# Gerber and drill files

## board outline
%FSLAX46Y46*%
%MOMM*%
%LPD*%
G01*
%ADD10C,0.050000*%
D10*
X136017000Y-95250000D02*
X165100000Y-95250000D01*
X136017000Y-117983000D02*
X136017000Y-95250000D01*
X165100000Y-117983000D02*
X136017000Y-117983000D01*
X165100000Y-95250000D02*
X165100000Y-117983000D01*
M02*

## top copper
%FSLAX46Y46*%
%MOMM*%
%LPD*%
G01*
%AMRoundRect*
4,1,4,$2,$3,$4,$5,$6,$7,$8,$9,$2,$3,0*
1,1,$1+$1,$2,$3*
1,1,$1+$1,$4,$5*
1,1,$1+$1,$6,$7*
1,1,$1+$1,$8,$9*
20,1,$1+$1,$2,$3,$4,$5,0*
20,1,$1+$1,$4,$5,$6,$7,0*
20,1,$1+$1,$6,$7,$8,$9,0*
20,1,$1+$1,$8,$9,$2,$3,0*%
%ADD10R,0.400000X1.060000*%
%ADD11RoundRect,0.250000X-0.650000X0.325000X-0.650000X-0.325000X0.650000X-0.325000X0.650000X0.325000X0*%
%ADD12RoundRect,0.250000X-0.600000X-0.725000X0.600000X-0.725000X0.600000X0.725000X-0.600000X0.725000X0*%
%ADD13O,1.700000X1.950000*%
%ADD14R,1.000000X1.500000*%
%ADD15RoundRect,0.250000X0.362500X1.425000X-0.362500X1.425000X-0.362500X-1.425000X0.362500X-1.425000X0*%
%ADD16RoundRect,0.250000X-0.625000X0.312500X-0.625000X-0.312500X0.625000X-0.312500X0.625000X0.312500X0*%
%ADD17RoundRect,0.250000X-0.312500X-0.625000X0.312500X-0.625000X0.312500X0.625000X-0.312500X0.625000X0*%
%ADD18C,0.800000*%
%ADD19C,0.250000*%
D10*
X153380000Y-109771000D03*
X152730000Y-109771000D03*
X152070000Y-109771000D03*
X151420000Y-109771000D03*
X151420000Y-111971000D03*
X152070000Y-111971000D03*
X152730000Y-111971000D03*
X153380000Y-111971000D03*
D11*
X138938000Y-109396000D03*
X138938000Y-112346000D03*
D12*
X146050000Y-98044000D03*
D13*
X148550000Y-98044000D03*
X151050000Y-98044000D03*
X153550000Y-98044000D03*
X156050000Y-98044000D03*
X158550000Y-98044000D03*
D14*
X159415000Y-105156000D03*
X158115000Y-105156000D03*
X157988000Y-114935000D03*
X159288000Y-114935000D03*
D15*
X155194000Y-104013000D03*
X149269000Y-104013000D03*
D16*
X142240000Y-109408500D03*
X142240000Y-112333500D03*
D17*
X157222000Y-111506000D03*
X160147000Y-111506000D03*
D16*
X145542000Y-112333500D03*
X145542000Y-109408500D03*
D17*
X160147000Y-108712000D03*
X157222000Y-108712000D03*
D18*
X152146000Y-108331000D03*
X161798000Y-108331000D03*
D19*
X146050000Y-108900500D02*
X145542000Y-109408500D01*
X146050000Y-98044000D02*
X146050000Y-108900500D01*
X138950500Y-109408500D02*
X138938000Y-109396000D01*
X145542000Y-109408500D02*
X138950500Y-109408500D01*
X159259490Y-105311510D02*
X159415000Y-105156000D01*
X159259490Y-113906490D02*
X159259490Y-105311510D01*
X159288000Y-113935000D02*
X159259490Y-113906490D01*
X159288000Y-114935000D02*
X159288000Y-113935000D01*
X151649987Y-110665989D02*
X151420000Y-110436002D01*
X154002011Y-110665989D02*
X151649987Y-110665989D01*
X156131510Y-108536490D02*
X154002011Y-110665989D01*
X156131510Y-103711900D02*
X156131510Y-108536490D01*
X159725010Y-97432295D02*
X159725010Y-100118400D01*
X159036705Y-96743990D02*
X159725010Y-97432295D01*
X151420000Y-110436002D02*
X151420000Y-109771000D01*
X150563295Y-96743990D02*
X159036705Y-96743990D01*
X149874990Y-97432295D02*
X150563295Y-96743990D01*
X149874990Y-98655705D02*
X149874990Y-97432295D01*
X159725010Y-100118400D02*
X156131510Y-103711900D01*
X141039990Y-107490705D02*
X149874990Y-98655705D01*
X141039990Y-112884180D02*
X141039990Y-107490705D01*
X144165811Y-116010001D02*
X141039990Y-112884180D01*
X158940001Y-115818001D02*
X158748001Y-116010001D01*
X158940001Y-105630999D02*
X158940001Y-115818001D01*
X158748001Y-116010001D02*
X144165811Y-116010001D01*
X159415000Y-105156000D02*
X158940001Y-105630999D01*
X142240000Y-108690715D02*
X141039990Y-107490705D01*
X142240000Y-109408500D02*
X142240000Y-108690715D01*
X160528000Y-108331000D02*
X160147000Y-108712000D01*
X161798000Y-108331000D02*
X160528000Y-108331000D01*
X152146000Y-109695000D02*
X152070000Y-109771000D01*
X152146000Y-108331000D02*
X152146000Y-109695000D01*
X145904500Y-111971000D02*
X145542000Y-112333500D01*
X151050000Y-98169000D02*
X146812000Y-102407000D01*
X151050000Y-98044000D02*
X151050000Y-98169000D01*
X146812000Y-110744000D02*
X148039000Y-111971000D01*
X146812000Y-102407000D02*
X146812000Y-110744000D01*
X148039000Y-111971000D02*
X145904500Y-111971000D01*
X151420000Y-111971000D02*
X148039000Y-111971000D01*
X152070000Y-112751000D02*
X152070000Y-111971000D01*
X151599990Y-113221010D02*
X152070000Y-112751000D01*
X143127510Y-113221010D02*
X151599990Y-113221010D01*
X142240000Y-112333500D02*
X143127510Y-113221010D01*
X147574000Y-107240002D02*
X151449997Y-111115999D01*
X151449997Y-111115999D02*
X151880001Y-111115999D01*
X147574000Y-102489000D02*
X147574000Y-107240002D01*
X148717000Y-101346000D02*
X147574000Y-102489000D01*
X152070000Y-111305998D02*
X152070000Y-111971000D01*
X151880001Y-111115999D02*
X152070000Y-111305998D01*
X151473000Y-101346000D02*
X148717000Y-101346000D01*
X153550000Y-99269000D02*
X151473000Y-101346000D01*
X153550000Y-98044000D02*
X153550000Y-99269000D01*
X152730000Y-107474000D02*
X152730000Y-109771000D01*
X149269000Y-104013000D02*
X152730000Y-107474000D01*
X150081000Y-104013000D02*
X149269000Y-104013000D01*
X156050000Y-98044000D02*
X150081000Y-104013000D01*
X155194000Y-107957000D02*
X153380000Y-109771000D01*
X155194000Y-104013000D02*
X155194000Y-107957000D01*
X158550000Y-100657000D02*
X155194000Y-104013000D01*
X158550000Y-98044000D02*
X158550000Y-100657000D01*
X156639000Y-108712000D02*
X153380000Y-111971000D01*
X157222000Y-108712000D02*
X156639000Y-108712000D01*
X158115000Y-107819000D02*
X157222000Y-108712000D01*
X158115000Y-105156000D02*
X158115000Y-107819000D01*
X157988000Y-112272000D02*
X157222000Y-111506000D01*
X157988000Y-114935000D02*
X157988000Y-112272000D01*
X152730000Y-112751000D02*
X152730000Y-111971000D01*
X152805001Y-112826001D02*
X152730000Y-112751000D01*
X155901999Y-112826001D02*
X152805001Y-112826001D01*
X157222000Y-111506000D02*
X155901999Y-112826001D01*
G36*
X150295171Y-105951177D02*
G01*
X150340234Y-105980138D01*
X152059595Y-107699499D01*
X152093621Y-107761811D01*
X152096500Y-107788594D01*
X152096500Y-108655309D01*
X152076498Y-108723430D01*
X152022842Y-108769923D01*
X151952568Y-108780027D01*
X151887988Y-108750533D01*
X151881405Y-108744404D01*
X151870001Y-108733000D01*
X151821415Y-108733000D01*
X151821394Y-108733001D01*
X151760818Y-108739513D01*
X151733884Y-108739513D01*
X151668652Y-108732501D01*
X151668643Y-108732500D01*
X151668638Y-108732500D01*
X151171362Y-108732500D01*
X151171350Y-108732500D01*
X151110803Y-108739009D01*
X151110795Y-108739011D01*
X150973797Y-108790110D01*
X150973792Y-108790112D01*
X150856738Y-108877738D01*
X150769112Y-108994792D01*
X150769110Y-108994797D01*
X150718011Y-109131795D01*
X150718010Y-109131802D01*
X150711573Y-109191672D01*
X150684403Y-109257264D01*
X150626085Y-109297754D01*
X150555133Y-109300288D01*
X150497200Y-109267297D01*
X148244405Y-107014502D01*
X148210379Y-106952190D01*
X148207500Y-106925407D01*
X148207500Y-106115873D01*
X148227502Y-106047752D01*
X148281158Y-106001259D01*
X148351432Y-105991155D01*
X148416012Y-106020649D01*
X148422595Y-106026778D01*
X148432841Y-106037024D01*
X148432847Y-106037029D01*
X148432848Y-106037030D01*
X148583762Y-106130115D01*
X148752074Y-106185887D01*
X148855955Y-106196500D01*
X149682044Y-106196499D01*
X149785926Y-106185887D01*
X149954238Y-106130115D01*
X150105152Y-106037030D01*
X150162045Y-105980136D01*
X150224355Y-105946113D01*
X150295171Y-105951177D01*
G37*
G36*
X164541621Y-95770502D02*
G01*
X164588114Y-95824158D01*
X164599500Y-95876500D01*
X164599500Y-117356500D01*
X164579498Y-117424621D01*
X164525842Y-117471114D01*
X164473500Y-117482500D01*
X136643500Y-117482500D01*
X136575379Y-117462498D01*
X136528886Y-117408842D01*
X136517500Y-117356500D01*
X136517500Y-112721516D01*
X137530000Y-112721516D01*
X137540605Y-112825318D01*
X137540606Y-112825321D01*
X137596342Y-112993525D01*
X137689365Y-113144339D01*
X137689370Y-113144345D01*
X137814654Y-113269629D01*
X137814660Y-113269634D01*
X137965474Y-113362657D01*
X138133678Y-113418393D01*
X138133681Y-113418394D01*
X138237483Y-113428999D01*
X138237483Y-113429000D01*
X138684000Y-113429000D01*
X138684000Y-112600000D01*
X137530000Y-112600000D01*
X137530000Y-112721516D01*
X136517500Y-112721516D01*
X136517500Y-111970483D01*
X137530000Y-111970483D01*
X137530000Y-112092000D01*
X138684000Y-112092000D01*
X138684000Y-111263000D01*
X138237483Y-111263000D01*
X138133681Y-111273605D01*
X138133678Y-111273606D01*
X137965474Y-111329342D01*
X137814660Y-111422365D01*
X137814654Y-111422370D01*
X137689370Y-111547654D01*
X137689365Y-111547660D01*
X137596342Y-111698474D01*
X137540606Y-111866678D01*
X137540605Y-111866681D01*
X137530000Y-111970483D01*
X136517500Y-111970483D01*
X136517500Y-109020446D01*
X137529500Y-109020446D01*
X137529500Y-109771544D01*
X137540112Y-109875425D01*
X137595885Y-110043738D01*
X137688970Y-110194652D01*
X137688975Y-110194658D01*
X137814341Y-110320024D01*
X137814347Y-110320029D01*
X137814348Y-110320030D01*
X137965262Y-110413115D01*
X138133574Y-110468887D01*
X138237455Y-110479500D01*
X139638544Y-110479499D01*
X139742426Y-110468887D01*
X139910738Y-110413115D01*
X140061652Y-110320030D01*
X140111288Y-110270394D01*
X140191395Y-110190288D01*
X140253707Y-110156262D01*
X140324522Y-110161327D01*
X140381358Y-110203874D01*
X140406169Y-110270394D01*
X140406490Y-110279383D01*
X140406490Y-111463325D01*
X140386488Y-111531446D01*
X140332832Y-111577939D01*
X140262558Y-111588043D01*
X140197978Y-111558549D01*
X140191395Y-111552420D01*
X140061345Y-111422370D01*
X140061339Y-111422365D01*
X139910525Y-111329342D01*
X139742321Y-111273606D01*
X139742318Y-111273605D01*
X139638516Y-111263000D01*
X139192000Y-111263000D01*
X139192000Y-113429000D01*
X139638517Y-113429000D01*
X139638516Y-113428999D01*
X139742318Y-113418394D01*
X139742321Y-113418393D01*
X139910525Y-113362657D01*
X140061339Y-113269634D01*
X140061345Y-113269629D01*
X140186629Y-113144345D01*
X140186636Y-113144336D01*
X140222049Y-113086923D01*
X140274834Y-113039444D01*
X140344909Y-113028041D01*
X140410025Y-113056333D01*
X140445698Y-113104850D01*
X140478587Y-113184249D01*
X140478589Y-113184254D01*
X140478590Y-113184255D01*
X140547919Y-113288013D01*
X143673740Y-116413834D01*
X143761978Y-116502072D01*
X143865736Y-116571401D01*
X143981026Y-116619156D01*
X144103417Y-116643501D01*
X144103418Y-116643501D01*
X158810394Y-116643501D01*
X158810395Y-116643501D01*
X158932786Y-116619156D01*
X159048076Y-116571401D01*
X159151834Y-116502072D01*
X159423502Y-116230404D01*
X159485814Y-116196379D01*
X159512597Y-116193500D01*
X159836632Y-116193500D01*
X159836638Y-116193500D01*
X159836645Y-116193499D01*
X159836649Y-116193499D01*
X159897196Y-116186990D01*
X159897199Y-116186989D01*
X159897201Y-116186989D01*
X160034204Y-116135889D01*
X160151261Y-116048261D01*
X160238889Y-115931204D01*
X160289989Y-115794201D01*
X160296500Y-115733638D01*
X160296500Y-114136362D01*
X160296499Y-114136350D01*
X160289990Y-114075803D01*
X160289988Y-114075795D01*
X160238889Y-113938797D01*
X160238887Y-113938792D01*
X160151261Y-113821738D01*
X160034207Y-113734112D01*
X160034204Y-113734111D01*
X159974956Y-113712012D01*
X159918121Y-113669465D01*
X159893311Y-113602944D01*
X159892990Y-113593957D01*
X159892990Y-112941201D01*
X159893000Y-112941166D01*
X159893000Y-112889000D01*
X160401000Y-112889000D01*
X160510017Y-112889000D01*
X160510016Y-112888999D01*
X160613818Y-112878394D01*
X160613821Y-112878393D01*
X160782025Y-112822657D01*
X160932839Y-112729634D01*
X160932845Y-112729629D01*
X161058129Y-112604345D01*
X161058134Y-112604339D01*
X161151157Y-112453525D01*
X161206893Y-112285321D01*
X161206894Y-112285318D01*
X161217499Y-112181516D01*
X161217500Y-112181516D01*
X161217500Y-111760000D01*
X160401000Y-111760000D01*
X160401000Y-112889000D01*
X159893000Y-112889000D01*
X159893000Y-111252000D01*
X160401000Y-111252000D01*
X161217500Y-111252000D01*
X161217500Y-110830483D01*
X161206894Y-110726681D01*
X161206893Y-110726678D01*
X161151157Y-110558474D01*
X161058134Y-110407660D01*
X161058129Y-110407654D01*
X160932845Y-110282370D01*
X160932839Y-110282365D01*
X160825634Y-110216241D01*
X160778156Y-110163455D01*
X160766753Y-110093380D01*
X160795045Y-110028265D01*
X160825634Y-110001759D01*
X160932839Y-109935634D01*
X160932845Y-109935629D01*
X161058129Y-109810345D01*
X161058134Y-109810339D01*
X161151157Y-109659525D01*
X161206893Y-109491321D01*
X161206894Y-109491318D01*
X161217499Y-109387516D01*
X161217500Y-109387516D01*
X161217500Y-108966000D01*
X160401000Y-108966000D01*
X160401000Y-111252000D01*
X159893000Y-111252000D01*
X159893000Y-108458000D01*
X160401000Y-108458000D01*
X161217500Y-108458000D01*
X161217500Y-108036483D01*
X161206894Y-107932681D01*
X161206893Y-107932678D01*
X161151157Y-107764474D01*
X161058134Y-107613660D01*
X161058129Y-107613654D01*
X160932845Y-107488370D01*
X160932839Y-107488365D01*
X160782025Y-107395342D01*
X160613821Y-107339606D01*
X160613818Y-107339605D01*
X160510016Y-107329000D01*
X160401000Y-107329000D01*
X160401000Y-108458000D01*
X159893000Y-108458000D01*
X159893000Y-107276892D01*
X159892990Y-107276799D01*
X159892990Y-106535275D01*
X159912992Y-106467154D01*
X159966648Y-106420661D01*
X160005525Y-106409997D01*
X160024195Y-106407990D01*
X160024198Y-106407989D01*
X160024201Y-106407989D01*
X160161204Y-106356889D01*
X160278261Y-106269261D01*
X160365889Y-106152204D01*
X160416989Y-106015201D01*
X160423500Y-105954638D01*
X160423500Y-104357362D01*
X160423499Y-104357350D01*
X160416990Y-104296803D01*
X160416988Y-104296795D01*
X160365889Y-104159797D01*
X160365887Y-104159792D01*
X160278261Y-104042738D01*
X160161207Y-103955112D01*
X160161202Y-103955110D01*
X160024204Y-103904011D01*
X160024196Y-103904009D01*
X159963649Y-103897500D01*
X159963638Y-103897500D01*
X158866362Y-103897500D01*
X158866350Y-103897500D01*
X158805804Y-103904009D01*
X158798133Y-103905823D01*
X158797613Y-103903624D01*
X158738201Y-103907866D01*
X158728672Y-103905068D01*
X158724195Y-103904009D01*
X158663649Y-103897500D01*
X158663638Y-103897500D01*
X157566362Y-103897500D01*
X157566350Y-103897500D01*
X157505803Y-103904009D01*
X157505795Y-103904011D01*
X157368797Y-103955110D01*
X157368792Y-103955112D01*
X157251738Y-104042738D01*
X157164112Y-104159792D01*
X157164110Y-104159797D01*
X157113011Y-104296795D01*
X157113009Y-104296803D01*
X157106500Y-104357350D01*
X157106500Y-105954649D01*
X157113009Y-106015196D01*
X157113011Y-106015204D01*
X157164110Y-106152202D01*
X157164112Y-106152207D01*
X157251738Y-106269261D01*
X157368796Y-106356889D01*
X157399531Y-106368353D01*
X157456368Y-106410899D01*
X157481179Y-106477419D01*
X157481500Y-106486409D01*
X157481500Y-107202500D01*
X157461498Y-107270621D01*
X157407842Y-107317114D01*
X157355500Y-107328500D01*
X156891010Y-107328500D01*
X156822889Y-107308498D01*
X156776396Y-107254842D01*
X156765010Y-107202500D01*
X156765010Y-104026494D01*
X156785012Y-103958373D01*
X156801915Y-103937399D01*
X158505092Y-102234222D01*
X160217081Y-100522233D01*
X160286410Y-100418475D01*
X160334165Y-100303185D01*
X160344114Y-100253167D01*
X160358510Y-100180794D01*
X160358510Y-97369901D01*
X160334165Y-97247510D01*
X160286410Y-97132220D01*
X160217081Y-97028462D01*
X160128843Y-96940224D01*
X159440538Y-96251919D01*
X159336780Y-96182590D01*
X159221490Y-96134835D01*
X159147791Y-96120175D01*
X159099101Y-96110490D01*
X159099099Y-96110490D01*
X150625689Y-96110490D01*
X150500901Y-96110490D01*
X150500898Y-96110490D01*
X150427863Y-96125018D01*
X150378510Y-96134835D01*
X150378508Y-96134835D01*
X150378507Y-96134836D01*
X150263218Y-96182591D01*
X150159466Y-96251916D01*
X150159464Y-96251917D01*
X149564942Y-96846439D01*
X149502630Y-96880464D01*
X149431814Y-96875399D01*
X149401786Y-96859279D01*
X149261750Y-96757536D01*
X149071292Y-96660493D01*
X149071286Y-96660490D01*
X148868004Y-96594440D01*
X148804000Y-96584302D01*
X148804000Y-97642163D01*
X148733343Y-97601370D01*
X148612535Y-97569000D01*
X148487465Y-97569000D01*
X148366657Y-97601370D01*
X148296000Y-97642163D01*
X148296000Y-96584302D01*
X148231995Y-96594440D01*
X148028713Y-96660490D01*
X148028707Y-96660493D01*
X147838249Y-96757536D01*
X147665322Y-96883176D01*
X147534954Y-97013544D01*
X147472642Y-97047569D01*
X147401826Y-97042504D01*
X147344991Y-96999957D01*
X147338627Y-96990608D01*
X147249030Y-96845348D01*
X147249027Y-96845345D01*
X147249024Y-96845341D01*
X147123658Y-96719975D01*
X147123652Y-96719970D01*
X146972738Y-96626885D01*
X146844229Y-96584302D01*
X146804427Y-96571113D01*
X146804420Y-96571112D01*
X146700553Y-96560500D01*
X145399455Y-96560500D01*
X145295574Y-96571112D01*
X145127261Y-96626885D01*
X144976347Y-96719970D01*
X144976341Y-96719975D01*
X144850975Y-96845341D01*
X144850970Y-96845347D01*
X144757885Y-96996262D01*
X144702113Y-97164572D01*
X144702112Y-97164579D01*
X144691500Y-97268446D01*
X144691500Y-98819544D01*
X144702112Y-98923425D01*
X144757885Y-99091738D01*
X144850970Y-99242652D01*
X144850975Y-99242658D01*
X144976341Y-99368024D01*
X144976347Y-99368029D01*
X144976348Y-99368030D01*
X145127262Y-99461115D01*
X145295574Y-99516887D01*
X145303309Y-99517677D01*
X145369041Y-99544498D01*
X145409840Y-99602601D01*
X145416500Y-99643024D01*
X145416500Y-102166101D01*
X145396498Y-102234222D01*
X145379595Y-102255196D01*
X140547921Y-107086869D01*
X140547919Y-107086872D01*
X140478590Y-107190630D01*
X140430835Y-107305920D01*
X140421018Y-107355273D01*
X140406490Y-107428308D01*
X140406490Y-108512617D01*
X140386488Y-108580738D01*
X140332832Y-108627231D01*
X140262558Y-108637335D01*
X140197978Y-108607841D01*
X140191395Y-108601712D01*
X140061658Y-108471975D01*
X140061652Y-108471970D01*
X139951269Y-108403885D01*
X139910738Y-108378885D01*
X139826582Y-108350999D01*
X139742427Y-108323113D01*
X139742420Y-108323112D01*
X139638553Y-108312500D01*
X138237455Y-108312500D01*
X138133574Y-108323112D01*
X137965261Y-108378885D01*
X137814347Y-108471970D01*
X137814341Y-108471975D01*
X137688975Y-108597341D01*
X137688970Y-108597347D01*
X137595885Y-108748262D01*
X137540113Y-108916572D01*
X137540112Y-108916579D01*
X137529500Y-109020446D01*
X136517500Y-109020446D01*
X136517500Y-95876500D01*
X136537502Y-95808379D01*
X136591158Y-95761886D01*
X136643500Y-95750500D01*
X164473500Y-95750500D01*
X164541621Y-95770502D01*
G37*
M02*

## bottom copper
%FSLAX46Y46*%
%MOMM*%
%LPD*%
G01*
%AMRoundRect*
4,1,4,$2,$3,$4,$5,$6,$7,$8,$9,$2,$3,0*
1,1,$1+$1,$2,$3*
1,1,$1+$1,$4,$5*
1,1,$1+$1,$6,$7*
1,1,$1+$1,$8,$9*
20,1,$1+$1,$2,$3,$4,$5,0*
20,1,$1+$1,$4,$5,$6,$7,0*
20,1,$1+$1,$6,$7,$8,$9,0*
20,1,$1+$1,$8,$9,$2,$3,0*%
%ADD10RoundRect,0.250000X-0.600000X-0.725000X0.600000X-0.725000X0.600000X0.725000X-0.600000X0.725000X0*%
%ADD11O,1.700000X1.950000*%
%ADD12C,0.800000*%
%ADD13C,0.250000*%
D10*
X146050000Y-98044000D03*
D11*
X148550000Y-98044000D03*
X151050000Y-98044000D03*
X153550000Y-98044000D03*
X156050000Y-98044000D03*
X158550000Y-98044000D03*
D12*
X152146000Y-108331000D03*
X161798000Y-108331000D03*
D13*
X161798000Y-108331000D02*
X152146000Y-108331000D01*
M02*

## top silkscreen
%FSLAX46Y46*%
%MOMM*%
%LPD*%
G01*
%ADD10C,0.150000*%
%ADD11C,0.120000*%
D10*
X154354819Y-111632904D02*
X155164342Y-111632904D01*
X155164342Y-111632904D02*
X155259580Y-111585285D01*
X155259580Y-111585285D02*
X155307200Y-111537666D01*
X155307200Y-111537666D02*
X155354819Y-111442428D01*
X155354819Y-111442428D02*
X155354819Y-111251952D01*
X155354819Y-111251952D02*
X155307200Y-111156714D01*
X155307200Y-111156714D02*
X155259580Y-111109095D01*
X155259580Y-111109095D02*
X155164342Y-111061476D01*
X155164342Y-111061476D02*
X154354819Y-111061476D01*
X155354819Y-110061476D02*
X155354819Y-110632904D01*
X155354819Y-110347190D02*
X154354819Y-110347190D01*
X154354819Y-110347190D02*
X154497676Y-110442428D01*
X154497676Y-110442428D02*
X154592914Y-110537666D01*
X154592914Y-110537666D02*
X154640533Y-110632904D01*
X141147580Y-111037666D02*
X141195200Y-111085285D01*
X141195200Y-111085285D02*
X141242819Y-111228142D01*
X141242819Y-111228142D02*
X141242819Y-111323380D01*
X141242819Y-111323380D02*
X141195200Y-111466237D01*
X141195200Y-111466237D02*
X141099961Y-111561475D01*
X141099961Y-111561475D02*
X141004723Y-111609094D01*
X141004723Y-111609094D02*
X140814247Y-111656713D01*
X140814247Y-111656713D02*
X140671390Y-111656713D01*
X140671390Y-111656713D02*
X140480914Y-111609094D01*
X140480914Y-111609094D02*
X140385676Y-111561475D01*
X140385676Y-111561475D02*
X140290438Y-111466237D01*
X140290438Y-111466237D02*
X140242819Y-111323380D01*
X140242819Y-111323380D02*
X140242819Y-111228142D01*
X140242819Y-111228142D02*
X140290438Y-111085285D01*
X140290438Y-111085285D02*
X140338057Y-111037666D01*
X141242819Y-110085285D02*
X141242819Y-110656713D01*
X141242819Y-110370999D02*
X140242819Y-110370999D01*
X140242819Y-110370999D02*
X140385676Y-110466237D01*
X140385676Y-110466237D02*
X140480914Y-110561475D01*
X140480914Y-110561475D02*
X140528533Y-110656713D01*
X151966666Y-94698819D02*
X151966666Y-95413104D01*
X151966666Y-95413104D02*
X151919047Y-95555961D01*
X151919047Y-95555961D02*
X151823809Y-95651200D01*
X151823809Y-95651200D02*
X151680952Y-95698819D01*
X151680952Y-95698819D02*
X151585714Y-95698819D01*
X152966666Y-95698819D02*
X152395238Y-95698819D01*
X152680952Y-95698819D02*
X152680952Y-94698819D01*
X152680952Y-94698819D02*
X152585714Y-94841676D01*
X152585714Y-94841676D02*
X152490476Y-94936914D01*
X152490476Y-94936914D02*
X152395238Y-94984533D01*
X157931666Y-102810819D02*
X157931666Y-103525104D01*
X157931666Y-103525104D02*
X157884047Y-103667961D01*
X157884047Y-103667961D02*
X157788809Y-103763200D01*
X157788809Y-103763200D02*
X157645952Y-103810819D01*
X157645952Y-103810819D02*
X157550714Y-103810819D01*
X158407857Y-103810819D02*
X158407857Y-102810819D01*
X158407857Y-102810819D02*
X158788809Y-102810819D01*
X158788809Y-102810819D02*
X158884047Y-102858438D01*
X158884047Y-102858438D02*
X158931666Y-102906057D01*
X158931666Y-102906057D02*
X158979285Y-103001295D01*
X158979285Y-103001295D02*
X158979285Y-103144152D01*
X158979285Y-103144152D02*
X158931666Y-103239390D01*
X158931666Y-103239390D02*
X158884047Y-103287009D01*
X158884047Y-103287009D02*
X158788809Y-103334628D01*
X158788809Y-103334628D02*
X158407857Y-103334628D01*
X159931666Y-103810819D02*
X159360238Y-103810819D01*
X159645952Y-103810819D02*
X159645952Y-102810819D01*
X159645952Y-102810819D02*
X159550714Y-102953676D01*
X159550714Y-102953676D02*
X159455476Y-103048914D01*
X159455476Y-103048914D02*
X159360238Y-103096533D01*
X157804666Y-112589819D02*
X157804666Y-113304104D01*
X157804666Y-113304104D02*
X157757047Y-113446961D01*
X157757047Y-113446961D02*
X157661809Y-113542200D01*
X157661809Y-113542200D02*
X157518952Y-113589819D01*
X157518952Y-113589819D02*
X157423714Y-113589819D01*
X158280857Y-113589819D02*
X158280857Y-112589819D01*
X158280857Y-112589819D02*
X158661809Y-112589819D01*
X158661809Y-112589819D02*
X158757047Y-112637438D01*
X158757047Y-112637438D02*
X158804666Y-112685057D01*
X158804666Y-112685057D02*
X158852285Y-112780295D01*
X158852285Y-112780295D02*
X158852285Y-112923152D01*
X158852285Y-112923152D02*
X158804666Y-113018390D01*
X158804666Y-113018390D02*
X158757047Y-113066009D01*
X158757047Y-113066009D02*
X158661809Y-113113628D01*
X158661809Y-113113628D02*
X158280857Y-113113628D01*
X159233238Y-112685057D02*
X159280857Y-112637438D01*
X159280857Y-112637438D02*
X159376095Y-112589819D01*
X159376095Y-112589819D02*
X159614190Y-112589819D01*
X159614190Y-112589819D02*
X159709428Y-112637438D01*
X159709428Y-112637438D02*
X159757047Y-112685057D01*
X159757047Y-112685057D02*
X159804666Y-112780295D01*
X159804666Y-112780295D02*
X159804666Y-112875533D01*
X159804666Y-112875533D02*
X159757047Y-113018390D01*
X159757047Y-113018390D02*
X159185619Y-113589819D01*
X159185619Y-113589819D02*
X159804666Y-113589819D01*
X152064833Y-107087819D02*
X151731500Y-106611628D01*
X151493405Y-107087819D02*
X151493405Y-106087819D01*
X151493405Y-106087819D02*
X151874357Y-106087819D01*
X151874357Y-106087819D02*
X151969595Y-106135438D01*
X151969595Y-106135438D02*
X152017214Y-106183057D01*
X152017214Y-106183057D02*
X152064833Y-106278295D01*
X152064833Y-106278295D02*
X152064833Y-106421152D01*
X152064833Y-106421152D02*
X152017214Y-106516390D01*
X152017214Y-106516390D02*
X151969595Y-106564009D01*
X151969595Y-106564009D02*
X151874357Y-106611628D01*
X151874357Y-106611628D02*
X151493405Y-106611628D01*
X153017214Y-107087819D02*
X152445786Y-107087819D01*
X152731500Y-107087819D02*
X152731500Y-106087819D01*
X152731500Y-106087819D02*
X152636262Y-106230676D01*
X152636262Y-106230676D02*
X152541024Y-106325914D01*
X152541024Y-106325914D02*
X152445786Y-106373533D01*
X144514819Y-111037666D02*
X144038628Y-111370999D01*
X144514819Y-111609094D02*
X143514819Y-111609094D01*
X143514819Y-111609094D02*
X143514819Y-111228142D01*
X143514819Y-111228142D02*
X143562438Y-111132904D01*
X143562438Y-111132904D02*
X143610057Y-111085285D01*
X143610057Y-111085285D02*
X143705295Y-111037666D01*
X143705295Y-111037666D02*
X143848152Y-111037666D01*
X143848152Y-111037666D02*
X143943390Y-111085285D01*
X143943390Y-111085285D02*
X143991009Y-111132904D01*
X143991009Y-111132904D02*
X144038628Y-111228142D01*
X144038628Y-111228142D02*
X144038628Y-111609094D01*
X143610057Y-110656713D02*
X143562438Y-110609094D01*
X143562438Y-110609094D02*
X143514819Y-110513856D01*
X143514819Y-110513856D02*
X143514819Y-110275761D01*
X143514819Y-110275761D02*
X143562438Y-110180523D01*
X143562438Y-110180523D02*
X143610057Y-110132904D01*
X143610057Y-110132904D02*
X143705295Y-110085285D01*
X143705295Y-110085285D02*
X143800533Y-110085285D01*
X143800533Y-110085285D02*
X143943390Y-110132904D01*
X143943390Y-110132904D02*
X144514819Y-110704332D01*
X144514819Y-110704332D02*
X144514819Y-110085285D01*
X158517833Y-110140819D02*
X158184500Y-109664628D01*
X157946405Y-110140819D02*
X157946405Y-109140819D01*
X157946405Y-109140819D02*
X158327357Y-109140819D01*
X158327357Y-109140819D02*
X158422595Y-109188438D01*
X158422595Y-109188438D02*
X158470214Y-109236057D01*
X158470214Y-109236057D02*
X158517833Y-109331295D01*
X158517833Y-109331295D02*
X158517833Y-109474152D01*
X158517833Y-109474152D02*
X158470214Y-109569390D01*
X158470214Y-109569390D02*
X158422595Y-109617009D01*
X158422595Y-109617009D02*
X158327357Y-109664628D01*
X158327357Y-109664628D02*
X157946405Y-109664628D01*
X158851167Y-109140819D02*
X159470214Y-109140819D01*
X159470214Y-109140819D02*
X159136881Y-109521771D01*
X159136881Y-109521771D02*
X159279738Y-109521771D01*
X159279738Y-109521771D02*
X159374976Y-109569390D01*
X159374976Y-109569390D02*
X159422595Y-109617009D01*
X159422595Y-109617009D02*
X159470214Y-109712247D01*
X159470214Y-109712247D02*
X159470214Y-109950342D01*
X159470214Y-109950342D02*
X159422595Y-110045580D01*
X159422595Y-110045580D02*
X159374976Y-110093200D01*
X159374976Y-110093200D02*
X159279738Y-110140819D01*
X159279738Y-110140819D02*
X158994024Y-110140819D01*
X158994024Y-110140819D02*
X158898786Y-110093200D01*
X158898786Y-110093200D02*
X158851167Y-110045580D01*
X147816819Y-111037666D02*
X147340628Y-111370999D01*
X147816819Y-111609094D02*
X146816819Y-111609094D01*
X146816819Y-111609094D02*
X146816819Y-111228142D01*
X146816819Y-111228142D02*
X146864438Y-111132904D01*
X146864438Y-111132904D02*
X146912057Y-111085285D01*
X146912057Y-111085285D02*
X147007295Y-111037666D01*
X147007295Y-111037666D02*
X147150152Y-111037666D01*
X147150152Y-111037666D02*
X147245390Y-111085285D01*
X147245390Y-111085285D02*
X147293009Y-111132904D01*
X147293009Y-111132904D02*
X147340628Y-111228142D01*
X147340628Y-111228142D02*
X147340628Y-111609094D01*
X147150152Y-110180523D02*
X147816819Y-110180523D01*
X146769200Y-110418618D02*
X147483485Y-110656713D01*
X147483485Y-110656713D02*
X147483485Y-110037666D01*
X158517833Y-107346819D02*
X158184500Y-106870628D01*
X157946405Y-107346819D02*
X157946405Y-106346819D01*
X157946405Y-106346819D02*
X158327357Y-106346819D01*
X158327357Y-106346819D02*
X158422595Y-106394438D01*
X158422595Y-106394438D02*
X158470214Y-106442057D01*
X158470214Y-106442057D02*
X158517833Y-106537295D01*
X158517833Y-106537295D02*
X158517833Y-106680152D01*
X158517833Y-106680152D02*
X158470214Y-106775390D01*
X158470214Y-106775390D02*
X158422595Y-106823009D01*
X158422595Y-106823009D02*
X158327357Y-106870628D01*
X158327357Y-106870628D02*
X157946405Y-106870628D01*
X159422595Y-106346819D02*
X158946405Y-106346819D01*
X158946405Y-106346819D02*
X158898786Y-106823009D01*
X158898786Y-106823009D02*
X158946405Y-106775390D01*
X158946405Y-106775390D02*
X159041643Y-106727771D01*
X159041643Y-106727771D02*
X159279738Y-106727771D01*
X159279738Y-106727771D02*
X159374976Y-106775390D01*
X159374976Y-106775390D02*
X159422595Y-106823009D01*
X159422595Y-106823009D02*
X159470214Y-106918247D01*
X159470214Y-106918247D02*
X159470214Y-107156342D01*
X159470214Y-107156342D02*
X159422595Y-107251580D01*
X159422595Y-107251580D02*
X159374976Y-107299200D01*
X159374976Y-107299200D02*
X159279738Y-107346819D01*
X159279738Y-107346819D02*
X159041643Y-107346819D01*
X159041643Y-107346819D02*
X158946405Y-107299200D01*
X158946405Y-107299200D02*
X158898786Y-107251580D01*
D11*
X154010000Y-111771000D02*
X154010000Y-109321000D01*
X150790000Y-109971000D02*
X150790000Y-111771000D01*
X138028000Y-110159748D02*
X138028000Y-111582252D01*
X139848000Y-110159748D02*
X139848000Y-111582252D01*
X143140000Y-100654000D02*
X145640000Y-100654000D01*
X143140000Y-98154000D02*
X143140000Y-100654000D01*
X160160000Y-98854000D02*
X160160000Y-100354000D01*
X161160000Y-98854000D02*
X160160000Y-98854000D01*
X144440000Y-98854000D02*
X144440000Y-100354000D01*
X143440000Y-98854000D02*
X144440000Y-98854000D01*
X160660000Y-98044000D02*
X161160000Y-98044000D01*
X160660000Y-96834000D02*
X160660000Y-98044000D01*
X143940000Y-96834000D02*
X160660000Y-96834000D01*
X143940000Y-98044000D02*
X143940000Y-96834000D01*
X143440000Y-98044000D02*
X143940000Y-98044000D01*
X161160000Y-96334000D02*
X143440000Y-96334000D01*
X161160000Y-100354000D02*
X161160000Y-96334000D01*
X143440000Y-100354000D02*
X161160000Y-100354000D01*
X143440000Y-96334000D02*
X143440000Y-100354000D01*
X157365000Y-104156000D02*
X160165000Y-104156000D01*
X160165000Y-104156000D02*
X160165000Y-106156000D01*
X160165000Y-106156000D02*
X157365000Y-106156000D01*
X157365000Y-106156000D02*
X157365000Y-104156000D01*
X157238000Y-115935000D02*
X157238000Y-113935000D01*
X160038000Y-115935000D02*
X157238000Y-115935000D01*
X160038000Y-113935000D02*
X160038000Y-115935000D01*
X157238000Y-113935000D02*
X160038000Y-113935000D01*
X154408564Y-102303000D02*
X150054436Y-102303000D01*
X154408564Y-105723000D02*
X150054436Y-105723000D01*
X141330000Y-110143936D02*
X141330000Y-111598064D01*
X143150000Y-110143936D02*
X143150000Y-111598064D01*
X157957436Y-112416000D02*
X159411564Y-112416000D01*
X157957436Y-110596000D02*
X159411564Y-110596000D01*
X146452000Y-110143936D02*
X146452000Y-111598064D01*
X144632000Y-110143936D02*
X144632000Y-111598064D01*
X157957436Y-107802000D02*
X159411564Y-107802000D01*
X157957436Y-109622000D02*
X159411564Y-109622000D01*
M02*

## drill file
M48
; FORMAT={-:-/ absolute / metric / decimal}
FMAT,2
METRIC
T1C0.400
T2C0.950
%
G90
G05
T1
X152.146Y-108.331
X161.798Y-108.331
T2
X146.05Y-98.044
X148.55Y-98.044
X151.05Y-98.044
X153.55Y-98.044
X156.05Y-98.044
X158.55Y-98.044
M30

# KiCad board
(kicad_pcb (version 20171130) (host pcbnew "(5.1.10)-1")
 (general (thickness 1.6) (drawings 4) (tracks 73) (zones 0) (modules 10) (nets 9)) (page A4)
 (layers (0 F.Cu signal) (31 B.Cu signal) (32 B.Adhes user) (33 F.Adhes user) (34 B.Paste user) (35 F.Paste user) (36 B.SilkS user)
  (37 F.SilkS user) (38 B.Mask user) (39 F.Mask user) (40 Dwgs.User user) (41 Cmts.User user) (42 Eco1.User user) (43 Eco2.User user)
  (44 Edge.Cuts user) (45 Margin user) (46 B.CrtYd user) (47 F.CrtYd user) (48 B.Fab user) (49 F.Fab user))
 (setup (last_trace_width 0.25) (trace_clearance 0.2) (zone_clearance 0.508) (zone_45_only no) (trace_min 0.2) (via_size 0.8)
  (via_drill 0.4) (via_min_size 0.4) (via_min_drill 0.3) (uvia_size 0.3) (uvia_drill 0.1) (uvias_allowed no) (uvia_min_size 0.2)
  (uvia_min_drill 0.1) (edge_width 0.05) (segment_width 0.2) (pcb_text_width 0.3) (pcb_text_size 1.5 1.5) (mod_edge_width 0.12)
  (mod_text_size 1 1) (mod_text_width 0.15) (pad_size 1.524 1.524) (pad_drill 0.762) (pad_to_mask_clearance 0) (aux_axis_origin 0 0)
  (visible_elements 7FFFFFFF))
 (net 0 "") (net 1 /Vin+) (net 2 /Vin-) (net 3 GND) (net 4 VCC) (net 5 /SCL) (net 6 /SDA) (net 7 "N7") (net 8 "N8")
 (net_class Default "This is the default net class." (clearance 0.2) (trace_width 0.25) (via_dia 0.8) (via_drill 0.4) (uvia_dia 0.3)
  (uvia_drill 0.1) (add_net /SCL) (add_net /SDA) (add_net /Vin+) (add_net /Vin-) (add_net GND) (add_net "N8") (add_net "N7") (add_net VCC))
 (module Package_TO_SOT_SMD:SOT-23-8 (layer F.Cu) (at 152.4 110.871 270)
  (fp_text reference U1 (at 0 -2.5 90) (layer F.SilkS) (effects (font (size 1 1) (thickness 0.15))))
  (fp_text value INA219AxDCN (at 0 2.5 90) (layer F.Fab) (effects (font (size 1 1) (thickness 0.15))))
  (fp_line (start 0.9 -1.61) (end -1.55 -1.61) (layer F.SilkS) (width 0.12))
  (fp_line (start -0.9 1.61) (end 0.9 1.61) (layer F.SilkS) (width 0.12))
  (pad 1 smd rect (at -1.1 -0.98 270) (size 1.06 0.4) (layers F.Cu F.Paste F.Mask) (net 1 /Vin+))
  (pad 2 smd rect (at -1.1 -0.33 270) (size 1.06 0.4) (layers F.Cu F.Paste F.Mask) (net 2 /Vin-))
  (pad 3 smd rect (at -1.1 0.33 270) (size 1.06 0.4) (layers F.Cu F.Paste F.Mask) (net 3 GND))
  (pad 4 smd rect (at -1.1 0.98 270) (size 1.06 0.4) (layers F.Cu F.Paste F.Mask) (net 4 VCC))
  (pad 5 smd rect (at 1.1 0.98 270) (size 1.06 0.4) (layers F.Cu F.Paste F.Mask) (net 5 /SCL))
  (pad 6 smd rect (at 1.1 0.33 270) (size 1.06 0.4) (layers F.Cu F.Paste F.Mask) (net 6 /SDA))
  (pad 7 smd rect (at 1.1 -0.33 270) (size 1.06 0.4) (layers F.Cu F.Paste F.Mask) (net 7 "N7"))
  (pad 8 smd rect (at 1.1 -0.98 270) (size 1.06 0.4) (layers F.Cu F.Paste F.Mask) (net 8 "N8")))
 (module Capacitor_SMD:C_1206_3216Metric (layer F.Cu) (at 138.938 110.871 270)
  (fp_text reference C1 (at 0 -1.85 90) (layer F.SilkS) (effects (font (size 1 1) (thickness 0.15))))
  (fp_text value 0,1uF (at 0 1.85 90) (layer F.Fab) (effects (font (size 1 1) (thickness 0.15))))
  (fp_line (start -0.711252 0.91) (end 0.711252 0.91) (layer F.SilkS) (width 0.12))
  (fp_line (start -0.711252 -0.91) (end 0.711252 -0.91) (layer F.SilkS) (width 0.12))
  (pad 1 smd roundrect (at -1.475 0 270) (size 1.15 1.8) (layers F.Cu F.Paste F.Mask) (roundrect_rratio 0.217391) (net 4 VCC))
  (pad 2 smd roundrect (at 1.475 0 270) (size 1.15 1.8) (layers F.Cu F.Paste F.Mask) (roundrect_rratio 0.217391) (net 3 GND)))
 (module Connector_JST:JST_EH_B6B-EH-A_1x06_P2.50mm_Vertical (layer F.Cu) (at 146.05 98.044)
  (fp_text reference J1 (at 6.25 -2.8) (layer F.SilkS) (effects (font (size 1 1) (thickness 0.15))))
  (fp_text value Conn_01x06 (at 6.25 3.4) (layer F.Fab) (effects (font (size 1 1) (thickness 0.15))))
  (fp_line (start -2.91 2.61) (end -0.41 2.61) (layer F.SilkS) (width 0.12))
  (fp_line (start -2.91 0.11) (end -2.91 2.61) (layer F.SilkS) (width 0.12))
  (fp_line (start 14.11 0.81) (end 14.11 2.31) (layer F.SilkS) (width 0.12))
  (fp_line (start 15.11 0.81) (end 14.11 0.81) (layer F.SilkS) (width 0.12))
  (fp_line (start -1.61 0.81) (end -1.61 2.31) (layer F.SilkS) (width 0.12))
  (fp_line (start -2.61 0.81) (end -1.61 0.81) (layer F.SilkS) (width 0.12))
  (fp_line (start 14.61 0) (end 15.11 0) (layer F.SilkS) (width 0.12))
  (fp_line (start 14.61 -1.21) (end 14.61 0) (layer F.SilkS) (width 0.12))
  (fp_line (start -2.11 -1.21) (end 14.61 -1.21) (layer F.SilkS) (width 0.12))
  (fp_line (start -2.11 0) (end -2.11 -1.21) (layer F.SilkS) (width 0.12))
  (fp_line (start -2.61 0) (end -2.11 0) (layer F.SilkS) (width 0.12))
  (fp_line (start 15.11 -1.71) (end -2.61 -1.71) (layer F.SilkS) (width 0.12))
  (fp_line (start 15.11 2.31) (end 15.11 -1.71) (layer F.SilkS) (width 0.12))
  (fp_line (start -2.61 2.31) (end 15.11 2.31) (layer F.SilkS) (width 0.12))
  (fp_line (start -2.61 -1.71) (end -2.61 2.31) (layer F.SilkS) (width 0.12))
  (pad 1 thru_hole roundrect (at 0 0) (size 1.7 1.95) (drill 0.95) (layers *.Cu *.Mask) (roundrect_rratio 0.147059) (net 4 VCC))
  (pad 2 thru_hole oval (at 2.5 0) (size 1.7 1.95) (drill 0.95) (layers *.Cu *.Mask) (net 3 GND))
  (pad 3 thru_hole oval (at 5 0) (size 1.7 1.95) (drill 0.95) (layers *.Cu *.Mask) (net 5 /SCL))
  (pad 4 thru_hole oval (at 7.5 0) (size 1.7 1.95) (drill 0.95) (layers *.Cu *.Mask) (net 6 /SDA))
  (pad 5 thru_hole oval (at 10 0) (size 1.7 1.95) (drill 0.95) (layers *.Cu *.Mask) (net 2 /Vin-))
  (pad 6 thru_hole oval (at 12.5 0) (size 1.7 1.95) (drill 0.95) (layers *.Cu *.Mask) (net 1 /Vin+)))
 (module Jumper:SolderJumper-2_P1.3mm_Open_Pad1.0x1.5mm (layer F.Cu) (at 158.765 105.156)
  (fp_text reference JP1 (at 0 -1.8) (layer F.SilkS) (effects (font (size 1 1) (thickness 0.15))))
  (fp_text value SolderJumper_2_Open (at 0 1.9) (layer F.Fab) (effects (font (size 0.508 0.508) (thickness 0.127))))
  (fp_line (start -1.4 -1) (end 1.4 -1) (layer F.SilkS) (width 0.12))
  (fp_line (start 1.4 -1) (end 1.4 1) (layer F.SilkS) (width 0.12))
  (fp_line (start 1.4 1) (end -1.4 1) (layer F.SilkS) (width 0.12))
  (fp_line (start -1.4 1) (end -1.4 -1) (layer F.SilkS) (width 0.12))
  (pad 2 smd rect (at 0.65 0) (size 1 1.5) (layers F.Cu F.Mask) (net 4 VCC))
  (pad 1 smd rect (at -0.65 0) (size 1 1.5) (layers F.Cu F.Mask) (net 8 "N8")))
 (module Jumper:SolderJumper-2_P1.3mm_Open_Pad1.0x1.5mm (layer F.Cu) (at 158.638 114.935)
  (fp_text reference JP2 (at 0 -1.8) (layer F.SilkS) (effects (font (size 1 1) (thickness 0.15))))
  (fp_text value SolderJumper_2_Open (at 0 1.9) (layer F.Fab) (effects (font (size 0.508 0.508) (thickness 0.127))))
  (fp_line (start -1.4 1) (end -1.4 -1) (layer F.SilkS) (width 0.12))
  (fp_line (start 1.4 1) (end -1.4 1) (layer F.SilkS) (width 0.12))
  (fp_line (start 1.4 -1) (end 1.4 1) (layer F.SilkS) (width 0.12))
  (fp_line (start -1.4 -1) (end 1.4 -1) (layer F.SilkS) (width 0.12))
  (pad 1 smd rect (at -0.65 0) (size 1 1.5) (layers F.Cu F.Mask) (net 7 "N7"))
  (pad 2 smd rect (at 0.65 0) (size 1 1.5) (layers F.Cu F.Mask) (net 4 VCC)))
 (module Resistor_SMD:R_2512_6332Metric (layer F.Cu) (at 152.2315 104.013 180)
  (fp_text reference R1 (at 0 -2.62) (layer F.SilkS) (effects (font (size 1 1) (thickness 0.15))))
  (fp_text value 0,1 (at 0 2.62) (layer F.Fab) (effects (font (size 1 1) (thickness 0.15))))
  (fp_line (start -2.177064 1.71) (end 2.177064 1.71) (layer F.SilkS) (width 0.12))
  (fp_line (start -2.177064 -1.71) (end 2.177064 -1.71) (layer F.SilkS) (width 0.12))
  (pad 1 smd roundrect (at -2.9625 0 180) (size 1.225 3.35) (layers F.Cu F.Paste F.Mask) (roundrect_rratio 0.204082) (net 1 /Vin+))
  (pad 2 smd roundrect (at 2.9625 0 180) (size 1.225 3.35) (layers F.Cu F.Paste F.Mask) (roundrect_rratio 0.204082) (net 2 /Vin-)))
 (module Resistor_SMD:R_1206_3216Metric (layer F.Cu) (at 142.24 110.871 270)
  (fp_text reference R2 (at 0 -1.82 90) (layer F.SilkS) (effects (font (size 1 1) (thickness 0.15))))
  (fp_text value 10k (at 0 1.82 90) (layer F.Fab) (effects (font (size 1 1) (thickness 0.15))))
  (fp_line (start -0.727064 0.91) (end 0.727064 0.91) (layer F.SilkS) (width 0.12))
  (fp_line (start -0.727064 -0.91) (end 0.727064 -0.91) (layer F.SilkS) (width 0.12))
  (pad 1 smd roundrect (at -1.4625 0 270) (size 1.125 1.75) (layers F.Cu F.Paste F.Mask) (roundrect_rratio 0.222222) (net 4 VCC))
  (pad 2 smd roundrect (at 1.4625 0 270) (size 1.125 1.75) (layers F.Cu F.Paste F.Mask) (roundrect_rratio 0.222222) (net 6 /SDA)))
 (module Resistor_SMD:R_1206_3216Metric (layer F.Cu) (at 158.6845 111.506)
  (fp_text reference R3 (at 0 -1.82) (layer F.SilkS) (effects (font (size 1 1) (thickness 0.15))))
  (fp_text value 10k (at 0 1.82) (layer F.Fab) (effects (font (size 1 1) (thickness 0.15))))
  (fp_line (start -0.727064 0.91) (end 0.727064 0.91) (layer F.SilkS) (width 0.12))
  (fp_line (start -0.727064 -0.91) (end 0.727064 -0.91) (layer F.SilkS) (width 0.12))
  (pad 1 smd roundrect (at -1.4625 0) (size 1.125 1.75) (layers F.Cu F.Paste F.Mask) (roundrect_rratio 0.222222) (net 7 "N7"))
  (pad 2 smd roundrect (at 1.4625 0) (size 1.125 1.75) (layers F.Cu F.Paste F.Mask) (roundrect_rratio 0.222222) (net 3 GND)))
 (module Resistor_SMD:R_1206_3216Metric (layer F.Cu) (at 145.542 110.871 270)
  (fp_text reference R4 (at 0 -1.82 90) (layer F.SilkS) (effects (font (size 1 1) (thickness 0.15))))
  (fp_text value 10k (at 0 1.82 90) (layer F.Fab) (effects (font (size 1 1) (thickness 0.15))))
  (fp_line (start -0.727064 -0.91) (end 0.727064 -0.91) (layer F.SilkS) (width 0.12))
  (fp_line (start -0.727064 0.91) (end 0.727064 0.91) (layer F.SilkS) (width 0.12))
  (pad 2 smd roundrect (at 1.4625 0 270) (size 1.125 1.75) (layers F.Cu F.Paste F.Mask) (roundrect_rratio 0.222222) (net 5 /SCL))
  (pad 1 smd roundrect (at -1.4625 0 270) (size 1.125 1.75) (layers F.Cu F.Paste F.Mask) (roundrect_rratio 0.222222) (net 4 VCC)))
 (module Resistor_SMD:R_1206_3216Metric (layer F.Cu) (at 158.6845 108.712)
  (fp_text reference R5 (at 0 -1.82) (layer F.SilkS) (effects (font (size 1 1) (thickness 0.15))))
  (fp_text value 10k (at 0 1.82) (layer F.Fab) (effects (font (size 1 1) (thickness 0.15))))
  (fp_line (start -0.727064 -0.91) (end 0.727064 -0.91) (layer F.SilkS) (width 0.12))
  (fp_line (start -0.727064 0.91) (end 0.727064 0.91) (layer F.SilkS) (width 0.12))
  (pad 2 smd roundrect (at 1.4625 0) (size 1.125 1.75) (layers F.Cu F.Paste F.Mask) (roundrect_rratio 0.222222) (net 3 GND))
  (pad 1 smd roundrect (at -1.4625 0) (size 1.125 1.75) (layers F.Cu F.Paste F.Mask) (roundrect_rratio 0.222222) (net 8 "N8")))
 (gr_line (start 136.017 95.25) (end 165.1 95.25) (layer Edge.Cuts) (width 0.05))
 (gr_line (start 136.017 117.983) (end 136.017 95.25) (layer Edge.Cuts) (width 0.05))
 (gr_line (start 165.1 117.983) (end 136.017 117.983) (layer Edge.Cuts) (width 0.05))
 (gr_line (start 165.1 95.25) (end 165.1 117.983) (layer Edge.Cuts) (width 0.05))
 (segment (start 146.05 108.9005) (end 145.542 109.4085) (width 0.25) (layer F.Cu) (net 4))
 (segment (start 146.05 98.044) (end 146.05 108.9005) (width 0.25) (layer F.Cu) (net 4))
 (segment (start 138.9505 109.4085) (end 138.938 109.396) (width 0.25) (layer F.Cu) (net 4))
 (segment (start 145.542 109.4085) (end 138.9505 109.4085) (width 0.25) (layer F.Cu) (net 4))
 (segment (start 159.25949 105.31151) (end 159.415 105.156) (width 0.25) (layer F.Cu) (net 4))
 (segment (start 159.25949 113.90649) (end 159.25949 105.31151) (width 0.25) (layer F.Cu) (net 4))
 (segment (start 159.288 113.935) (end 159.25949 113.90649) (width 0.25) (layer F.Cu) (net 4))
 (segment (start 159.288 114.935) (end 159.288 113.935) (width 0.25) (layer F.Cu) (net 4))
 (segment (start 151.649987 110.665989) (end 151.42 110.436002) (width 0.25) (layer F.Cu) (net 4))
 (segment (start 154.002011 110.665989) (end 151.649987 110.665989) (width 0.25) (layer F.Cu) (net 4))
 (segment (start 156.13151 108.53649) (end 154.002011 110.665989) (width 0.25) (layer F.Cu) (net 4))
 (segment (start 156.13151 103.7119) (end 156.13151 108.53649) (width 0.25) (layer F.Cu) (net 4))
 (segment (start 159.72501 97.432295) (end 159.72501 100.1184) (width 0.25) (layer F.Cu) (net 4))
 (segment (start 159.036705 96.74399) (end 159.72501 97.432295) (width 0.25) (layer F.Cu) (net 4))
 (segment (start 151.42 110.436002) (end 151.42 109.771) (width 0.25) (layer F.Cu) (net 4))
 (segment (start 150.563295 96.74399) (end 159.036705 96.74399) (width 0.25) (layer F.Cu) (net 4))
 (segment (start 149.87499 97.432295) (end 150.563295 96.74399) (width 0.25) (layer F.Cu) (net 4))
 (segment (start 149.87499 98.655705) (end 149.87499 97.432295) (width 0.25) (layer F.Cu) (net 4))
 (segment (start 159.72501 100.1184) (end 156.13151 103.7119) (width 0.25) (layer F.Cu) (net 4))
 (segment (start 141.03999 107.490705) (end 149.87499 98.655705) (width 0.25) (layer F.Cu) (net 4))
 (segment (start 141.03999 112.88418) (end 141.03999 107.490705) (width 0.25) (layer F.Cu) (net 4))
 (segment (start 144.165811 116.010001) (end 141.03999 112.88418) (width 0.25) (layer F.Cu) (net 4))
 (segment (start 158.940001 115.818001) (end 158.748001 116.010001) (width 0.25) (layer F.Cu) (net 4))
 (segment (start 158.940001 105.630999) (end 158.940001 115.818001) (width 0.25) (layer F.Cu) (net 4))
 (segment (start 158.748001 116.010001) (end 144.165811 116.010001) (width 0.25) (layer F.Cu) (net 4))
 (segment (start 159.415 105.156) (end 158.940001 105.630999) (width 0.25) (layer F.Cu) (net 4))
 (segment (start 142.24 108.690715) (end 141.03999 107.490705) (width 0.25) (layer F.Cu) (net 4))
 (segment (start 142.24 109.4085) (end 142.24 108.690715) (width 0.25) (layer F.Cu) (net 4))
 (via (at 152.146 108.331) (size 0.8) (drill 0.4) (layers F.Cu B.Cu) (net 3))
 (via (at 161.798 108.331) (size 0.8) (drill 0.4) (layers F.Cu B.Cu) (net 3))
 (segment (start 160.528 108.331) (end 160.147 108.712) (width 0.25) (layer F.Cu) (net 3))
 (segment (start 161.798 108.331) (end 160.528 108.331) (width 0.25) (layer F.Cu) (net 3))
 (segment (start 161.798 108.331) (end 152.146 108.331) (width 0.25) (layer B.Cu) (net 3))
 (segment (start 152.146 109.695) (end 152.07 109.771) (width 0.25) (layer F.Cu) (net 3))
 (segment (start 152.146 108.331) (end 152.146 109.695) (width 0.25) (layer F.Cu) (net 3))
 (segment (start 145.9045 111.971) (end 145.542 112.3335) (width 0.25) (layer F.Cu) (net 5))
 (segment (start 151.05 98.169) (end 146.812 102.407) (width 0.25) (layer F.Cu) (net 5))
 (segment (start 151.05 98.044) (end 151.05 98.169) (width 0.25) (layer F.Cu) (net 5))
 (segment (start 146.812 110.744) (end 148.039 111.971) (width 0.25) (layer F.Cu) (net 5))
 (segment (start 146.812 102.407) (end 146.812 110.744) (width 0.25) (layer F.Cu) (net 5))
 (segment (start 148.039 111.971) (end 145.9045 111.971) (width 0.25) (layer F.Cu) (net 5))
 (segment (start 151.42 111.971) (end 148.039 111.971) (width 0.25) (layer F.Cu) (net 5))
 (segment (start 152.07 112.751) (end 152.07 111.971) (width 0.25) (layer F.Cu) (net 6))
 (segment (start 151.59999 113.22101) (end 152.07 112.751) (width 0.25) (layer F.Cu) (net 6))
 (segment (start 143.12751 113.22101) (end 151.59999 113.22101) (width 0.25) (layer F.Cu) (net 6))
 (segment (start 142.24 112.3335) (end 143.12751 113.22101) (width 0.25) (layer F.Cu) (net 6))
 (segment (start 147.574 107.240002) (end 151.449997 111.115999) (width 0.25) (layer F.Cu) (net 6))
 (segment (start 151.449997 111.115999) (end 151.880001 111.115999) (width 0.25) (layer F.Cu) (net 6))
 (segment (start 147.574 102.489) (end 147.574 107.240002) (width 0.25) (layer F.Cu) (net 6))
 (segment (start 148.717 101.346) (end 147.574 102.489) (width 0.25) (layer F.Cu) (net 6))
 (segment (start 152.07 111.305998) (end 152.07 111.971) (width 0.25) (layer F.Cu) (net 6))
 (segment (start 151.880001 111.115999) (end 152.07 111.305998) (width 0.25) (layer F.Cu) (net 6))
 (segment (start 151.473 101.346) (end 148.717 101.346) (width 0.25) (layer F.Cu) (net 6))
 (segment (start 153.55 99.269) (end 151.473 101.346) (width 0.25) (layer F.Cu) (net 6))
 (segment (start 153.55 98.044) (end 153.55 99.269) (width 0.25) (layer F.Cu) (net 6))
 (segment (start 152.73 107.474) (end 152.73 109.771) (width 0.25) (layer F.Cu) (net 2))
 (segment (start 149.269 104.013) (end 152.73 107.474) (width 0.25) (layer F.Cu) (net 2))
 (segment (start 150.081 104.013) (end 149.269 104.013) (width 0.25) (layer F.Cu) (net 2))
 (segment (start 156.05 98.044) (end 150.081 104.013) (width 0.25) (layer F.Cu) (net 2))
 (segment (start 155.194 107.957) (end 153.38 109.771) (width 0.25) (layer F.Cu) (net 1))
 (segment (start 155.194 104.013) (end 155.194 107.957) (width 0.25) (layer F.Cu) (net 1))
 (segment (start 158.55 100.657) (end 155.194 104.013) (width 0.25) (layer F.Cu) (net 1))
 (segment (start 158.55 98.044) (end 158.55 100.657) (width 0.25) (layer F.Cu) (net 1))
 (segment (start 156.639 108.712) (end 153.38 111.971) (width 0.25) (layer F.Cu) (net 8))
 (segment (start 157.222 108.712) (end 156.639 108.712) (width 0.25) (layer F.Cu) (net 8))
 (segment (start 158.115 107.819) (end 157.222 108.712) (width 0.25) (layer F.Cu) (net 8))
 (segment (start 158.115 105.156) (end 158.115 107.819) (width 0.25) (layer F.Cu) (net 8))
 (segment (start 157.988 112.272) (end 157.222 111.506) (width 0.25) (layer F.Cu) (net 7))
 (segment (start 157.988 114.935) (end 157.988 112.272) (width 0.25) (layer F.Cu) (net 7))
 (segment (start 152.73 112.751) (end 152.73 111.971) (width 0.25) (layer F.Cu) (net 7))
 (segment (start 152.805001 112.826001) (end 152.73 112.751) (width 0.25) (layer F.Cu) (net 7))
 (segment (start 155.901999 112.826001) (end 152.805001 112.826001) (width 0.25) (layer F.Cu) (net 7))
 (segment (start 157.222 111.506) (end 155.901999 112.826001) (width 0.25) (layer F.Cu) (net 7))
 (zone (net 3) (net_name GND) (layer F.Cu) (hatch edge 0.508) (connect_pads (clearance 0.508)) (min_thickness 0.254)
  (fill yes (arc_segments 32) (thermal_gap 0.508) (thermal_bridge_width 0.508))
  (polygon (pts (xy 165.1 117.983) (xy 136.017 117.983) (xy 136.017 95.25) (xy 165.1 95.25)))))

